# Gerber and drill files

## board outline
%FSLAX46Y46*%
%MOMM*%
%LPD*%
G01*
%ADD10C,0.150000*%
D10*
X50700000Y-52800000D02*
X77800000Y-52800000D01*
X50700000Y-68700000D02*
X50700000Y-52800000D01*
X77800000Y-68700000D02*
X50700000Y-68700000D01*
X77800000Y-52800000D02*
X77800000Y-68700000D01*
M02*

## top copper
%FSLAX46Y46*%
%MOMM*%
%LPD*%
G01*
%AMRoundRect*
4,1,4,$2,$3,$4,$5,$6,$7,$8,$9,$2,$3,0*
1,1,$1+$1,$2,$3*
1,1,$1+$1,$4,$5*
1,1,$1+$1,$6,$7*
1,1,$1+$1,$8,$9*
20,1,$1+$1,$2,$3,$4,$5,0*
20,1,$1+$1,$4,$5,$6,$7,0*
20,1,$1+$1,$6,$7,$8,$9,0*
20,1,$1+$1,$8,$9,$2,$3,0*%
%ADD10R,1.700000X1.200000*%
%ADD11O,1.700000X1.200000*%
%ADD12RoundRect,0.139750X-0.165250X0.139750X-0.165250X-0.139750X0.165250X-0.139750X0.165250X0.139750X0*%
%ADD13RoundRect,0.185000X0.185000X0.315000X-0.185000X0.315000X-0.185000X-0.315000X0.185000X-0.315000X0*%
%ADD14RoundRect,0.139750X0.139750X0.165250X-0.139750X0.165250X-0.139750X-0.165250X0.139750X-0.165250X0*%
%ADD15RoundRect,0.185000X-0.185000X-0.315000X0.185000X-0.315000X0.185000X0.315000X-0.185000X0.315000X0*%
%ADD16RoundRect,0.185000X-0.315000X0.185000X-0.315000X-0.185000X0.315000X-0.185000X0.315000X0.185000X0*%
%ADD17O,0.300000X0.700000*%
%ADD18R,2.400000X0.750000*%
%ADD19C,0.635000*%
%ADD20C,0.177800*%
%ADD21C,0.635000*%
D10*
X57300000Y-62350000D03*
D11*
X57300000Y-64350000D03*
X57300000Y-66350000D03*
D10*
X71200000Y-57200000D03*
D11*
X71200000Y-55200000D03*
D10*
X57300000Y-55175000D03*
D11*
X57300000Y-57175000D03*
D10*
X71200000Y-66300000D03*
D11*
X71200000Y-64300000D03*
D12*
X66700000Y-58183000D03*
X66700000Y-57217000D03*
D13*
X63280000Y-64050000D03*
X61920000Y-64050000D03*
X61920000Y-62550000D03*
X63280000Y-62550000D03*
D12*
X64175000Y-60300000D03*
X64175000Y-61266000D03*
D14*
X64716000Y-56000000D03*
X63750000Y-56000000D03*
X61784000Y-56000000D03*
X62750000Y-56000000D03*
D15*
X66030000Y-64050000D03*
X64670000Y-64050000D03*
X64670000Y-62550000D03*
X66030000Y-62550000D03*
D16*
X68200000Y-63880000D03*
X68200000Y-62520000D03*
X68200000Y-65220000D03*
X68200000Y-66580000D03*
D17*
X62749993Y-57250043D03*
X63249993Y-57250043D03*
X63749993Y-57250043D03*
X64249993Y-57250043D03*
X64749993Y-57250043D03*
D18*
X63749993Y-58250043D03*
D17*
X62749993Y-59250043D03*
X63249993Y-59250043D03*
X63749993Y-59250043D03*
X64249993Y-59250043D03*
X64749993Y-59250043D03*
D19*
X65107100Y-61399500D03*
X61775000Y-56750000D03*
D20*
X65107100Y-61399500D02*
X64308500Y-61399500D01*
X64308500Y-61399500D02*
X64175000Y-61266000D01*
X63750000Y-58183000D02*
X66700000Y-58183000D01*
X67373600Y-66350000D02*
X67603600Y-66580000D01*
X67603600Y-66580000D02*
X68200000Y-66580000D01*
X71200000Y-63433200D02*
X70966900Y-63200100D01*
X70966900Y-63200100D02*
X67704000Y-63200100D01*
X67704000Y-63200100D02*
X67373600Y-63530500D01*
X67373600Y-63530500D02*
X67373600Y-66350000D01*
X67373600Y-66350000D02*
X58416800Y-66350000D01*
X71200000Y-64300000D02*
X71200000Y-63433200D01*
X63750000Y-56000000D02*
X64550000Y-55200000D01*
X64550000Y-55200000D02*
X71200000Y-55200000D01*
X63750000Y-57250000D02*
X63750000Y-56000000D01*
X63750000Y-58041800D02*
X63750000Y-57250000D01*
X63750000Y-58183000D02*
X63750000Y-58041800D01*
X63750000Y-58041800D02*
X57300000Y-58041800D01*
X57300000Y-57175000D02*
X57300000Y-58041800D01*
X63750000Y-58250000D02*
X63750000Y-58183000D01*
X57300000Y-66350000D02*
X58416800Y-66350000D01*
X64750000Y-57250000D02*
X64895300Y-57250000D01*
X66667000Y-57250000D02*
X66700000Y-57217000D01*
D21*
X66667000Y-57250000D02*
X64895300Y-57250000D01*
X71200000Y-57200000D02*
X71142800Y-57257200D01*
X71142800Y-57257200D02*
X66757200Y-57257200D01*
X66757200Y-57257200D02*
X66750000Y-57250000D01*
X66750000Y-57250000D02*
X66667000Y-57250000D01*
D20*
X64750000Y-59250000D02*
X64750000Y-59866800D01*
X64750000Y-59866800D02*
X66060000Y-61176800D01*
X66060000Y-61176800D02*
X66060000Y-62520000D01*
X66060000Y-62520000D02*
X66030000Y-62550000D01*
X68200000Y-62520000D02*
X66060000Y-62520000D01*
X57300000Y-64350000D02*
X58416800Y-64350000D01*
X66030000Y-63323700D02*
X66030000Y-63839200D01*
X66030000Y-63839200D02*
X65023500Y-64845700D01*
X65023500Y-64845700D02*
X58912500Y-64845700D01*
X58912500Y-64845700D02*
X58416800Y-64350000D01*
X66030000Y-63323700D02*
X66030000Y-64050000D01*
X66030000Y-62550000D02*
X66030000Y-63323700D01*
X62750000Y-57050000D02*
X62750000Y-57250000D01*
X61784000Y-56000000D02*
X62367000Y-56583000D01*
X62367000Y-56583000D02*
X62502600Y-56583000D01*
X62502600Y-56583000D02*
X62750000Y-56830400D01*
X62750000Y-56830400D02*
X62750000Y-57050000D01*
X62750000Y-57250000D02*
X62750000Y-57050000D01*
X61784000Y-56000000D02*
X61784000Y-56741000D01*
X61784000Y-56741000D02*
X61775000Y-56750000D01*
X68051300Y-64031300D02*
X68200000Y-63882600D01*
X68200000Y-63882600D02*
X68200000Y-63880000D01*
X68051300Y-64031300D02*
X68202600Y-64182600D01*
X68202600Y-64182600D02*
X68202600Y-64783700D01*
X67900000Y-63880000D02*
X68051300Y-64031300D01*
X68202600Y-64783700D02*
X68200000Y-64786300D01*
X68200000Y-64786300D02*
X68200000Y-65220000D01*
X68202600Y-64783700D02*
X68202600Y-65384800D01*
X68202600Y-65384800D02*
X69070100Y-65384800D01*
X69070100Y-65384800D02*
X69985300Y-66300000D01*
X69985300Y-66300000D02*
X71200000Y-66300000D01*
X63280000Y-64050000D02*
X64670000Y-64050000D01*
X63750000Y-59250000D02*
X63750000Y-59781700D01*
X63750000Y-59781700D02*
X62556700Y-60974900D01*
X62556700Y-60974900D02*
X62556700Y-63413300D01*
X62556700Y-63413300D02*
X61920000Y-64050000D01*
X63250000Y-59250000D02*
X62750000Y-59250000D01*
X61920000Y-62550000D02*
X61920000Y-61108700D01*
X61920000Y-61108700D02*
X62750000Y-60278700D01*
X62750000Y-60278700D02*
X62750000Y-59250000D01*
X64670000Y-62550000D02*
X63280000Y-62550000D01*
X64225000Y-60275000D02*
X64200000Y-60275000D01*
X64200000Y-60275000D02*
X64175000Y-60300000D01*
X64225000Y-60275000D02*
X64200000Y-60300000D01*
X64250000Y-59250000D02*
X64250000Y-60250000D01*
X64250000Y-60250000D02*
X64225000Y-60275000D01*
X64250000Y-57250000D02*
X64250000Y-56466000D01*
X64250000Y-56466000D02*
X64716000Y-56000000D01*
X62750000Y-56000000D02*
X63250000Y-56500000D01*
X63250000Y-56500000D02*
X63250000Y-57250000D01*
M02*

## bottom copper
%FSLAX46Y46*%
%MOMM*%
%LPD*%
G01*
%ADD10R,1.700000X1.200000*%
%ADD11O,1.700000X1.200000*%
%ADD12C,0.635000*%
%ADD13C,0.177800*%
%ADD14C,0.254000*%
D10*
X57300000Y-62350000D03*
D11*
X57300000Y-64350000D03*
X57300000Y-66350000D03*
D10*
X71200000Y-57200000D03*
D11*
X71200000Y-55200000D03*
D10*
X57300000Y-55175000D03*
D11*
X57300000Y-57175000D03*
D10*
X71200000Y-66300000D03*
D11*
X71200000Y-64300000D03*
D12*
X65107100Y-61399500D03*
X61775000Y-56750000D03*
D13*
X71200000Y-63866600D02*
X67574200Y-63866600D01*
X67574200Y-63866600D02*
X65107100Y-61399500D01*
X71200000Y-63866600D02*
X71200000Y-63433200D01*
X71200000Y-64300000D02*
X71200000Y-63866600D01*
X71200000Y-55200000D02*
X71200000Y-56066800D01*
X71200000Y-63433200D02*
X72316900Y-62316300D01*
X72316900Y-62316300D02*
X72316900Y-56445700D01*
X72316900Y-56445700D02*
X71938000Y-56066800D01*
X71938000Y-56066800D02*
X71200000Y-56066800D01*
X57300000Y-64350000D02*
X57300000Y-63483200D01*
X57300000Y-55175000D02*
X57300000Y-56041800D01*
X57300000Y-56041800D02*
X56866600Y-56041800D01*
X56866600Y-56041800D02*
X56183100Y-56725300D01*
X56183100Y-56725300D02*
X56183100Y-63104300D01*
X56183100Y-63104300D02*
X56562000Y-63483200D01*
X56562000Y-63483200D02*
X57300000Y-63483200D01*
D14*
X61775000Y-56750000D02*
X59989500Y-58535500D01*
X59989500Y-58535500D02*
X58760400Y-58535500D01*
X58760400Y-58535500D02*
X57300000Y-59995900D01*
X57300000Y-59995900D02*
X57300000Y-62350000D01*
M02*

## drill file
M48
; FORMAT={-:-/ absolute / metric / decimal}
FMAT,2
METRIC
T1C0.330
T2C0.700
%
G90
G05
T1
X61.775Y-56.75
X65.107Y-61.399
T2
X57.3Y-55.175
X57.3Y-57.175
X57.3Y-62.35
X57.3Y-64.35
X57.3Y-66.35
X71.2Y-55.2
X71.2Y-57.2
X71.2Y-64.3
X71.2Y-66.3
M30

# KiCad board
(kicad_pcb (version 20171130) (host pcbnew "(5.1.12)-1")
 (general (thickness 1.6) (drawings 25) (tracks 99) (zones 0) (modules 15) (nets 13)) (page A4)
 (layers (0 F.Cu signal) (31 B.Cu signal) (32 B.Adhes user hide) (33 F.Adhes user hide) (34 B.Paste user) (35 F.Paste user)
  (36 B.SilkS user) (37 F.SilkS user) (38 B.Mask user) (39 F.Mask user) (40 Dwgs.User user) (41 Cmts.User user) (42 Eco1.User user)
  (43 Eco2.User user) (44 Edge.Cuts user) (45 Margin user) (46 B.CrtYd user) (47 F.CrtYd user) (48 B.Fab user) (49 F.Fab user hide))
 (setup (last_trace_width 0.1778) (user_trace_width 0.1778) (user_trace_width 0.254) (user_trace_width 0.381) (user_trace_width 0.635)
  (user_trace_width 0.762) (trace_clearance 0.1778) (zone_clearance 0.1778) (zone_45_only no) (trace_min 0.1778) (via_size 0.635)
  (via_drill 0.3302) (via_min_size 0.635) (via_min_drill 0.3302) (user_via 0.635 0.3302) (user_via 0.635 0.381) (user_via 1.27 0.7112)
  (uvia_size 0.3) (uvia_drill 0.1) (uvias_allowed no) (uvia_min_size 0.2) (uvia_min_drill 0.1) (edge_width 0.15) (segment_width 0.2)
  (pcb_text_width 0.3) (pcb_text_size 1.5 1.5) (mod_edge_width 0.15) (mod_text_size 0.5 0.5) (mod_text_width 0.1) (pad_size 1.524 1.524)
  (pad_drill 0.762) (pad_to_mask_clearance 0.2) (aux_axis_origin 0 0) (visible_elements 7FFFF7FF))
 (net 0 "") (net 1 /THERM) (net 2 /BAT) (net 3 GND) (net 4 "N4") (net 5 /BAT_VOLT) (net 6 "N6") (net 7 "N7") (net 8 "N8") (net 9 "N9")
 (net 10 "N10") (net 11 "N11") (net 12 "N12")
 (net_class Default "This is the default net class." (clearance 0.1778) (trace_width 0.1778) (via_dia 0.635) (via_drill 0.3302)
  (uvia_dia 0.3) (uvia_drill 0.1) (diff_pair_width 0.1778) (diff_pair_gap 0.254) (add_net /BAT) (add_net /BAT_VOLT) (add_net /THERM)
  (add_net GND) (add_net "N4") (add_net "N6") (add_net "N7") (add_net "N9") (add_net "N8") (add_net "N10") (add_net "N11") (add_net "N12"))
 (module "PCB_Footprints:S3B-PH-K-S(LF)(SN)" (layer F.Cu) (at 57.3 62.35 270)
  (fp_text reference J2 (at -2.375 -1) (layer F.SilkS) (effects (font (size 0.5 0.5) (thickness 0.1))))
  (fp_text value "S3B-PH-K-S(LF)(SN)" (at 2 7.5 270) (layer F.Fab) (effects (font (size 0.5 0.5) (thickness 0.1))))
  (pad 1 thru_hole rect (at 0 0 270) (size 1.2 1.7) (drill 0.7) (layers *.Cu *.Mask F.SilkS) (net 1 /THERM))
  (pad 2 thru_hole oval (at 2 0 270) (size 1.2 1.7) (drill 0.7) (layers *.Cu *.Mask F.SilkS) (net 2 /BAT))
  (pad 3 thru_hole oval (at 4 0 270) (size 1.2 1.7) (drill 0.7) (layers *.Cu *.Mask F.SilkS) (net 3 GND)))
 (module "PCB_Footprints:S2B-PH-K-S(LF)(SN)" (layer F.Cu) (at 71.2 57.2 90)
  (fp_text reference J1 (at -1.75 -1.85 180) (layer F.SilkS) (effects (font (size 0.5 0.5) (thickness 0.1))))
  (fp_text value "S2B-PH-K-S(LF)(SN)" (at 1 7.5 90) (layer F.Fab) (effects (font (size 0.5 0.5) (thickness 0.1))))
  (pad 1 thru_hole rect (at 0 0 90) (size 1.2 1.7) (drill 0.7) (layers *.Cu *.Mask F.SilkS) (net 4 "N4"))
  (pad 2 thru_hole oval (at 2 0 90) (size 1.2 1.7) (drill 0.7) (layers *.Cu *.Mask F.SilkS) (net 3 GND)))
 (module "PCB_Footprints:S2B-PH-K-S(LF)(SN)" (layer F.Cu) (at 57.3 55.175 270)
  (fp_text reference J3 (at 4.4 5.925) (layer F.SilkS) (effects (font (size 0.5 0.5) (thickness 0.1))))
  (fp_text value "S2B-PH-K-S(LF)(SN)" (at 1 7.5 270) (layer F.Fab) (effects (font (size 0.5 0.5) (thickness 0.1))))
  (pad 1 thru_hole rect (at 0 0 270) (size 1.2 1.7) (drill 0.7) (layers *.Cu *.Mask F.SilkS) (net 2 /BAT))
  (pad 2 thru_hole oval (at 2 0 270) (size 1.2 1.7) (drill 0.7) (layers *.Cu *.Mask F.SilkS) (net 3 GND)))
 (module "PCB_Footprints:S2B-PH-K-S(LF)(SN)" (layer F.Cu) (at 71.2 66.3 90)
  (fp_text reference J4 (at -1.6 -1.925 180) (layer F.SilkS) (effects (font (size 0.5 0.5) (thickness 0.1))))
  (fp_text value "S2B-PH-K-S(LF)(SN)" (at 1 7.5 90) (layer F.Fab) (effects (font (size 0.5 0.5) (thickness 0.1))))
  (pad 1 thru_hole rect (at 0 0 90) (size 1.2 1.7) (drill 0.7) (layers *.Cu *.Mask F.SilkS) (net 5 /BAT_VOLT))
  (pad 2 thru_hole oval (at 2 0 90) (size 1.2 1.7) (drill 0.7) (layers *.Cu *.Mask F.SilkS) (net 3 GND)))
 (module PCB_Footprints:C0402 (layer F.Cu) (at 66.7 57.7 270)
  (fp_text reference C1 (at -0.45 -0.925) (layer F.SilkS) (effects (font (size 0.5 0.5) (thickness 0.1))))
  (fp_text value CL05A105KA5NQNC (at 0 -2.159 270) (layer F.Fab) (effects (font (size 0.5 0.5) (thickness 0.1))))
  (pad 2 smd roundrect (at 0.483 0 270) (size 0.559 0.61) (layers F.Cu F.Paste F.Mask) (roundrect_rratio 0.25) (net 3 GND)
   (solder_mask_margin 0.102))
  (pad 1 smd roundrect (at -0.483 0 270) (size 0.559 0.61) (layers F.Cu F.Paste F.Mask) (roundrect_rratio 0.25) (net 4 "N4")
   (solder_mask_margin 0.102)))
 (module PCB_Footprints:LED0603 (layer F.Cu) (at 62.6 64.05 180)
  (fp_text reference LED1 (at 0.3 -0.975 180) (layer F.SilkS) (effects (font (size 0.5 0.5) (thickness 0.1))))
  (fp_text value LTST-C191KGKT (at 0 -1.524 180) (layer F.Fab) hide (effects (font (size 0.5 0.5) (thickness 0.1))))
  (pad 1 smd roundrect (at -0.68 0 180) (size 0.74 1) (layers F.Cu F.Paste F.Mask) (roundrect_rratio 0.25) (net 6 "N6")
   (solder_mask_margin 0.102))
  (pad 2 smd roundrect (at 0.68 0 180) (size 0.74 1) (layers F.Cu F.Paste F.Mask) (roundrect_rratio 0.25) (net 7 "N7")
   (solder_mask_margin 0.102)))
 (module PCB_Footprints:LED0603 (layer F.Cu) (at 62.6 62.55 180)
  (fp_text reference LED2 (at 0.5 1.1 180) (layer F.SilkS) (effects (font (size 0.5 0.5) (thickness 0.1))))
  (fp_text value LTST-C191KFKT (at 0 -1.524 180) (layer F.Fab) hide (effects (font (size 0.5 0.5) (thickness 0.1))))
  (pad 2 smd roundrect (at 0.68 0 180) (size 0.74 1) (layers F.Cu F.Paste F.Mask) (roundrect_rratio 0.25) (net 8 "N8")
   (solder_mask_margin 0.102))
  (pad 1 smd roundrect (at -0.68 0 180) (size 0.74 1) (layers F.Cu F.Paste F.Mask) (roundrect_rratio 0.25) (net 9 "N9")
   (solder_mask_margin 0.102)))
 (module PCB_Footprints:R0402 (layer F.Cu) (at 64.175 60.783 270)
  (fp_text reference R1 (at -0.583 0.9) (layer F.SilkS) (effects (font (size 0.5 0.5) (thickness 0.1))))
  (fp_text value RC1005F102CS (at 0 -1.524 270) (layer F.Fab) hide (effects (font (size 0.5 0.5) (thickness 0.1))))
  (pad 1 smd roundrect (at -0.483 0 270) (size 0.559 0.61) (layers F.Cu F.Paste F.Mask) (roundrect_rratio 0.25) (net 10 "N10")
   (solder_mask_margin 0.102))
  (pad 2 smd roundrect (at 0.483 0 270) (size 0.559 0.61) (layers F.Cu F.Paste F.Mask) (roundrect_rratio 0.25) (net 3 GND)
   (solder_mask_margin 0.102)))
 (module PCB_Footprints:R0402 (layer F.Cu) (at 64.233 56 180)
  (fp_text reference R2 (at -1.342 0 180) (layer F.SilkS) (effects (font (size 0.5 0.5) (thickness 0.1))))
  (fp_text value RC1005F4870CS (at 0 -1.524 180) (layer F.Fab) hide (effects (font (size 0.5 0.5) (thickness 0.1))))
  (pad 1 smd roundrect (at -0.483 0 180) (size 0.559 0.61) (layers F.Cu F.Paste F.Mask) (roundrect_rratio 0.25) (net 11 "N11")
   (solder_mask_margin 0.102))
  (pad 2 smd roundrect (at 0.483 0 180) (size 0.559 0.61) (layers F.Cu F.Paste F.Mask) (roundrect_rratio 0.25) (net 3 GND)
   (solder_mask_margin 0.102)))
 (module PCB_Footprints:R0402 (layer F.Cu) (at 62.267 56 180)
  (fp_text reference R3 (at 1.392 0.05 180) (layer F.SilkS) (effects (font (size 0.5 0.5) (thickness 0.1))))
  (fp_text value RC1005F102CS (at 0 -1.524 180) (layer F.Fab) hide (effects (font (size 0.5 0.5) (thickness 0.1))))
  (pad 2 smd roundrect (at 0.483 0 180) (size 0.559 0.61) (layers F.Cu F.Paste F.Mask) (roundrect_rratio 0.25) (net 1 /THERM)
   (solder_mask_margin 0.102))
  (pad 1 smd roundrect (at -0.483 0 180) (size 0.559 0.61) (layers F.Cu F.Paste F.Mask) (roundrect_rratio 0.25) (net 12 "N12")
   (solder_mask_margin 0.102)))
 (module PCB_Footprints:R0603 (layer F.Cu) (at 65.35 64.05)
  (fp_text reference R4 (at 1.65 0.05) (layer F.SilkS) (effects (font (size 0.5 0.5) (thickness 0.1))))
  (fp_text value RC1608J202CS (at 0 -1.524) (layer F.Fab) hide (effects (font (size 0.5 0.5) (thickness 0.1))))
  (pad 2 smd roundrect (at 0.68 0) (size 0.74 1) (layers F.Cu F.Paste F.Mask) (roundrect_rratio 0.25) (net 2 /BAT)
   (solder_mask_margin 0.102))
  (pad 1 smd roundrect (at -0.68 0) (size 0.74 1) (layers F.Cu F.Paste F.Mask) (roundrect_rratio 0.25) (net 6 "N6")
   (solder_mask_margin 0.102)))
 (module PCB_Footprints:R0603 (layer F.Cu) (at 65.35 62.55)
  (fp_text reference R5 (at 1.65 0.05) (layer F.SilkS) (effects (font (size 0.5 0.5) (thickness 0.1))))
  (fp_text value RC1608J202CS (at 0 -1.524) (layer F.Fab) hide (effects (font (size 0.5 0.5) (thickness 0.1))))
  (pad 1 smd roundrect (at -0.68 0) (size 0.74 1) (layers F.Cu F.Paste F.Mask) (roundrect_rratio 0.25) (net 9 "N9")
   (solder_mask_margin 0.102))
  (pad 2 smd roundrect (at 0.68 0) (size 0.74 1) (layers F.Cu F.Paste F.Mask) (roundrect_rratio 0.25) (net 2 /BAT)
   (solder_mask_margin 0.102)))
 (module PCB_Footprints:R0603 (layer F.Cu) (at 68.2 63.2 270)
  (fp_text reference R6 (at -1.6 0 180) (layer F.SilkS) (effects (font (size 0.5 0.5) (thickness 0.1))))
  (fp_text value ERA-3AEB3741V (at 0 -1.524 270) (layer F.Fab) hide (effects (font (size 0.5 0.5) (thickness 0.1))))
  (pad 2 smd roundrect (at 0.68 0 270) (size 0.74 1) (layers F.Cu F.Paste F.Mask) (roundrect_rratio 0.25) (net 5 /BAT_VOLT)
   (solder_mask_margin 0.102))
  (pad 1 smd roundrect (at -0.68 0 270) (size 0.74 1) (layers F.Cu F.Paste F.Mask) (roundrect_rratio 0.25) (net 2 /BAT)
   (solder_mask_margin 0.102)))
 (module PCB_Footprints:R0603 (layer F.Cu) (at 68.2 65.9 270)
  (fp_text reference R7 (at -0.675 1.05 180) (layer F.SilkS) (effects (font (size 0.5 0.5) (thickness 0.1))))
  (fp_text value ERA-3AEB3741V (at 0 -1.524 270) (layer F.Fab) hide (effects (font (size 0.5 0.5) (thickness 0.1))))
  (pad 1 smd roundrect (at -0.68 0 270) (size 0.74 1) (layers F.Cu F.Paste F.Mask) (roundrect_rratio 0.25) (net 5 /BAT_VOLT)
   (solder_mask_margin 0.102))
  (pad 2 smd roundrect (at 0.68 0 270) (size 0.74 1) (layers F.Cu F.Paste F.Mask) (roundrect_rratio 0.25) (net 3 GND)
   (solder_mask_margin 0.102)))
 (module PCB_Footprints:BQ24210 (layer F.Cu) (at 63.7368 58.3252 270)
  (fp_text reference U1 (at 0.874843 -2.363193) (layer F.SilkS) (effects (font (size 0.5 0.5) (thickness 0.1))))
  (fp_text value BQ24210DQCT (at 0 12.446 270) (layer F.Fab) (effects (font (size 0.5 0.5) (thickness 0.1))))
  (pad 5 smd oval (at -1.075157 0.986807 180) (size 0.3 0.7) (layers F.Cu F.Paste F.Mask) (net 1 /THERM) (solder_mask_margin 0.102))
  (pad 4 smd oval (at -1.075157 0.486807 180) (size 0.3 0.7) (layers F.Cu F.Paste F.Mask) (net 12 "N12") (solder_mask_margin 0.102))
  (pad 3 smd oval (at -1.075157 -0.013193 180) (size 0.3 0.7) (layers F.Cu F.Paste F.Mask) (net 3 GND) (solder_mask_margin 0.102))
  (pad 2 smd oval (at -1.075157 -0.513193 180) (size 0.3 0.7) (layers F.Cu F.Paste F.Mask) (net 11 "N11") (solder_mask_margin 0.102))
  (pad 1 smd oval (at -1.075157 -1.013193 180) (size 0.3 0.7) (layers F.Cu F.Paste F.Mask) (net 4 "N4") (solder_mask_margin 0.102))
  (pad 11 smd rect (at -0.075157 -0.013193 180) (size 2.4 0.75) (layers F.Cu F.Paste F.Mask) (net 3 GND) (solder_mask_margin 0.102))
  (pad 6 smd oval (at 0.924843 0.986807 180) (size 0.3 0.7) (layers F.Cu F.Paste F.Mask) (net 8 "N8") (solder_mask_margin 0.102))
  (pad 7 smd oval (at 0.924843 0.486807 180) (size 0.3 0.7) (layers F.Cu F.Paste F.Mask) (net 8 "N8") (solder_mask_margin 0.102))
  (pad 8 smd oval (at 0.924843 -0.013193 180) (size 0.3 0.7) (layers F.Cu F.Paste F.Mask) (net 7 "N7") (solder_mask_margin 0.102))
  (pad 9 smd oval (at 0.924843 -0.513193 180) (size 0.3 0.7) (layers F.Cu F.Paste F.Mask) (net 10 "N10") (solder_mask_margin 0.102))
  (pad 10 smd oval (at 0.924843 -1.013193 180) (size 0.3 0.7) (layers F.Cu F.Paste F.Mask) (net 2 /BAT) (solder_mask_margin 0.102)))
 (gr_line (start 50.7 52.8) (end 77.8 52.8) (layer Edge.Cuts) (width 0.15))
 (gr_line (start 50.7 68.7) (end 50.7 52.8) (layer Edge.Cuts) (width 0.15))
 (gr_line (start 77.8 68.7) (end 50.7 68.7) (layer Edge.Cuts) (width 0.15))
 (gr_line (start 77.8 52.8) (end 77.8 68.7) (layer Edge.Cuts) (width 0.15))
 (segment (start 65.1071 61.3995) (end 64.3085 61.3995) (width 0.1778) (layer F.Cu) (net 3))
 (segment (start 64.3085 61.3995) (end 64.175 61.266) (width 0.1778) (layer F.Cu) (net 3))
 (segment (start 71.2 63.8666) (end 67.5742 63.8666) (width 0.1778) (layer B.Cu) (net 3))
 (segment (start 67.5742 63.8666) (end 65.1071 61.3995) (width 0.1778) (layer B.Cu) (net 3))
 (segment (start 71.2 63.8666) (end 71.2 63.4332) (width 0.1778) (layer B.Cu) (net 3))
 (segment (start 71.2 64.3) (end 71.2 63.8666) (width 0.1778) (layer B.Cu) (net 3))
 (segment (start 63.75 58.183) (end 66.7 58.183) (width 0.1778) (layer F.Cu) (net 3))
 (segment (start 67.3736 66.35) (end 67.6036 66.58) (width 0.1778) (layer F.Cu) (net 3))
 (segment (start 67.6036 66.58) (end 68.2 66.58) (width 0.1778) (layer F.Cu) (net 3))
 (segment (start 71.2 63.4332) (end 70.9669 63.2001) (width 0.1778) (layer F.Cu) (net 3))
 (segment (start 70.9669 63.2001) (end 67.704 63.2001) (width 0.1778) (layer F.Cu) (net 3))
 (segment (start 67.704 63.2001) (end 67.3736 63.5305) (width 0.1778) (layer F.Cu) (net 3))
 (segment (start 67.3736 63.5305) (end 67.3736 66.35) (width 0.1778) (layer F.Cu) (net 3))
 (segment (start 67.3736 66.35) (end 58.4168 66.35) (width 0.1778) (layer F.Cu) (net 3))
 (segment (start 71.2 64.3) (end 71.2 63.4332) (width 0.1778) (layer F.Cu) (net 3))
 (segment (start 63.75 56) (end 64.55 55.2) (width 0.1778) (layer F.Cu) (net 3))
 (segment (start 64.55 55.2) (end 71.2 55.2) (width 0.1778) (layer F.Cu) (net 3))
 (segment (start 63.75 57.25) (end 63.75 56) (width 0.1778) (layer F.Cu) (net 3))
 (segment (start 71.2 55.2) (end 71.2 56.0668) (width 0.1778) (layer B.Cu) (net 3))
 (segment (start 71.2 63.4332) (end 72.3169 62.3163) (width 0.1778) (layer B.Cu) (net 3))
 (segment (start 72.3169 62.3163) (end 72.3169 56.4457) (width 0.1778) (layer B.Cu) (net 3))
 (segment (start 72.3169 56.4457) (end 71.938 56.0668) (width 0.1778) (layer B.Cu) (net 3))
 (segment (start 71.938 56.0668) (end 71.2 56.0668) (width 0.1778) (layer B.Cu) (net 3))
 (segment (start 63.75 58.0418) (end 63.75 57.25) (width 0.1778) (layer F.Cu) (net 3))
 (segment (start 63.75 58.183) (end 63.75 58.0418) (width 0.1778) (layer F.Cu) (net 3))
 (segment (start 63.75 58.0418) (end 57.3 58.0418) (width 0.1778) (layer F.Cu) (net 3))
 (segment (start 57.3 57.175) (end 57.3 58.0418) (width 0.1778) (layer F.Cu) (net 3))
 (segment (start 63.75 58.25) (end 63.75 58.183) (width 0.1778) (layer F.Cu) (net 3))
 (segment (start 57.3 66.35) (end 58.4168 66.35) (width 0.1778) (layer F.Cu) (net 3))
 (via (at 65.1071 61.3995) (size 0.635) (layers F.Cu B.Cu) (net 3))
 (segment (start 64.75 57.25) (end 64.8953 57.25) (width 0.1778) (layer F.Cu) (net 4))
 (segment (start 66.667 57.25) (end 66.7 57.217) (width 0.1778) (layer F.Cu) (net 4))
 (segment (start 66.667 57.25) (end 64.8953 57.25) (width 0.635) (layer F.Cu) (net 4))
 (segment (start 71.2 57.2) (end 71.1428 57.2572) (width 0.635) (layer F.Cu) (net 4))
 (segment (start 71.1428 57.2572) (end 66.7572 57.2572) (width 0.635) (layer F.Cu) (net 4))
 (segment (start 66.7572 57.2572) (end 66.75 57.25) (width 0.635) (layer F.Cu) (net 4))
 (segment (start 66.75 57.25) (end 66.667 57.25) (width 0.635) (layer F.Cu) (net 4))
 (segment (start 64.75 59.25) (end 64.75 59.8668) (width 0.1778) (layer F.Cu) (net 2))
 (segment (start 64.75 59.8668) (end 66.06 61.1768) (width 0.1778) (layer F.Cu) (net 2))
 (segment (start 66.06 61.1768) (end 66.06 62.52) (width 0.1778) (layer F.Cu) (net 2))
 (segment (start 66.06 62.52) (end 66.03 62.55) (width 0.1778) (layer F.Cu) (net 2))
 (segment (start 68.2 62.52) (end 66.06 62.52) (width 0.1778) (layer F.Cu) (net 2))
 (segment (start 57.3 64.35) (end 57.3 63.4832) (width 0.1778) (layer B.Cu) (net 2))
 (segment (start 57.3 55.175) (end 57.3 56.0418) (width 0.1778) (layer B.Cu) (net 2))
 (segment (start 57.3 56.0418) (end 56.8666 56.0418) (width 0.1778) (layer B.Cu) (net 2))
 (segment (start 56.8666 56.0418) (end 56.1831 56.7253) (width 0.1778) (layer B.Cu) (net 2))
 (segment (start 56.1831 56.7253) (end 56.1831 63.1043) (width 0.1778) (layer B.Cu) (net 2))
 (segment (start 56.1831 63.1043) (end 56.562 63.4832) (width 0.1778) (layer B.Cu) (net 2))
 (segment (start 56.562 63.4832) (end 57.3 63.4832) (width 0.1778) (layer B.Cu) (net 2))
 (segment (start 57.3 64.35) (end 58.4168 64.35) (width 0.1778) (layer F.Cu) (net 2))
 (segment (start 66.03 63.3237) (end 66.03 63.8392) (width 0.1778) (layer F.Cu) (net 2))
 (segment (start 66.03 63.8392) (end 65.0235 64.8457) (width 0.1778) (layer F.Cu) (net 2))
 (segment (start 65.0235 64.8457) (end 58.9125 64.8457) (width 0.1778) (layer F.Cu) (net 2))
 (segment (start 58.9125 64.8457) (end 58.4168 64.35) (width 0.1778) (layer F.Cu) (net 2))
 (segment (start 66.03 63.3237) (end 66.03 64.05) (width 0.1778) (layer F.Cu) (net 2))
 (segment (start 66.03 62.55) (end 66.03 63.3237) (width 0.1778) (layer F.Cu) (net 2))
 (segment (start 62.75 57.05) (end 62.75 57.25) (width 0.1778) (layer F.Cu) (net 1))
 (segment (start 61.784 56) (end 62.367 56.583) (width 0.1778) (layer F.Cu) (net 1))
 (segment (start 62.367 56.583) (end 62.5026 56.583) (width 0.1778) (layer F.Cu) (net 1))
 (segment (start 62.5026 56.583) (end 62.75 56.8304) (width 0.1778) (layer F.Cu) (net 1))
 (segment (start 62.75 56.8304) (end 62.75 57.05) (width 0.1778) (layer F.Cu) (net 1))
 (segment (start 62.75 57.25) (end 62.75 57.05) (width 0.1778) (layer F.Cu) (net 1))
 (segment (start 61.784 56) (end 61.784 56.741) (width 0.1778) (layer F.Cu) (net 1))
 (segment (start 61.784 56.741) (end 61.775 56.75) (width 0.1778) (layer F.Cu) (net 1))
 (segment (start 61.775 56.75) (end 59.9895 58.5355) (width 0.254) (layer B.Cu) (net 1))
 (segment (start 59.9895 58.5355) (end 58.7604 58.5355) (width 0.254) (layer B.Cu) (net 1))
 (segment (start 58.7604 58.5355) (end 57.3 59.9959) (width 0.254) (layer B.Cu) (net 1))
 (segment (start 57.3 59.9959) (end 57.3 62.35) (width 0.254) (layer B.Cu) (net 1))
 (via (at 61.775 56.75) (size 0.635) (layers F.Cu B.Cu) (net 1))
 (segment (start 68.0513 64.0313) (end 68.2 63.8826) (width 0.1778) (layer F.Cu) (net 5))
 (segment (start 68.2 63.8826) (end 68.2 63.88) (width 0.1778) (layer F.Cu) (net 5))
 (segment (start 68.0513 64.0313) (end 68.2026 64.1826) (width 0.1778) (layer F.Cu) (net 5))
 (segment (start 68.2026 64.1826) (end 68.2026 64.7837) (width 0.1778) (layer F.Cu) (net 5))
 (segment (start 67.9 63.88) (end 68.0513 64.0313) (width 0.1778) (layer F.Cu) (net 5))
 (segment (start 68.2026 64.7837) (end 68.2 64.7863) (width 0.1778) (layer F.Cu) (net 5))
 (segment (start 68.2 64.7863) (end 68.2 65.22) (width 0.1778) (layer F.Cu) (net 5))
 (segment (start 68.2026 64.7837) (end 68.2026 65.3848) (width 0.1778) (layer F.Cu) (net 5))
 (segment (start 68.2026 65.3848) (end 69.0701 65.3848) (width 0.1778) (layer F.Cu) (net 5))
 (segment (start 69.0701 65.3848) (end 69.9853 66.3) (width 0.1778) (layer F.Cu) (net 5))
 (segment (start 69.9853 66.3) (end 71.2 66.3) (width 0.1778) (layer F.Cu) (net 5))
 (segment (start 63.28 64.05) (end 64.67 64.05) (width 0.1778) (layer F.Cu) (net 6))
 (segment (start 63.75 59.25) (end 63.75 59.7817) (width 0.1778) (layer F.Cu) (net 7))
 (segment (start 63.75 59.7817) (end 62.5567 60.9749) (width 0.1778) (layer F.Cu) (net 7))
 (segment (start 62.5567 60.9749) (end 62.5567 63.4133) (width 0.1778) (layer F.Cu) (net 7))
 (segment (start 62.5567 63.4133) (end 61.92 64.05) (width 0.1778) (layer F.Cu) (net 7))
 (segment (start 63.25 59.25) (end 62.75 59.25) (width 0.1778) (layer F.Cu) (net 8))
 (segment (start 61.92 62.55) (end 61.92 61.1087) (width 0.1778) (layer F.Cu) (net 8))
 (segment (start 61.92 61.1087) (end 62.75 60.2787) (width 0.1778) (layer F.Cu) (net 8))
 (segment (start 62.75 60.2787) (end 62.75 59.25) (width 0.1778) (layer F.Cu) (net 8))
 (segment (start 64.67 62.55) (end 63.28 62.55) (width 0.1778) (layer F.Cu) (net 9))
 (segment (start 64.225 60.275) (end 64.2 60.275) (width 0.1778) (layer F.Cu) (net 10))
 (segment (start 64.2 60.275) (end 64.175 60.3) (width 0.1778) (layer F.Cu) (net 10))
 (segment (start 64.225 60.275) (end 64.2 60.3) (width 0.1778) (layer F.Cu) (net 10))
 (segment (start 64.25 59.25) (end 64.25 60.25) (width 0.1778) (layer F.Cu) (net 10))
 (segment (start 64.25 60.25) (end 64.225 60.275) (width 0.1778) (layer F.Cu) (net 10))
 (segment (start 64.25 57.25) (end 64.25 56.466) (width 0.1778) (layer F.Cu) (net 11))
 (segment (start 64.25 56.466) (end 64.716 56) (width 0.1778) (layer F.Cu) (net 11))
 (segment (start 62.75 56) (end 63.25 56.5) (width 0.1778) (layer F.Cu) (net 12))
 (segment (start 63.25 56.5) (end 63.25 57.25) (width 0.1778) (layer F.Cu) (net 12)))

